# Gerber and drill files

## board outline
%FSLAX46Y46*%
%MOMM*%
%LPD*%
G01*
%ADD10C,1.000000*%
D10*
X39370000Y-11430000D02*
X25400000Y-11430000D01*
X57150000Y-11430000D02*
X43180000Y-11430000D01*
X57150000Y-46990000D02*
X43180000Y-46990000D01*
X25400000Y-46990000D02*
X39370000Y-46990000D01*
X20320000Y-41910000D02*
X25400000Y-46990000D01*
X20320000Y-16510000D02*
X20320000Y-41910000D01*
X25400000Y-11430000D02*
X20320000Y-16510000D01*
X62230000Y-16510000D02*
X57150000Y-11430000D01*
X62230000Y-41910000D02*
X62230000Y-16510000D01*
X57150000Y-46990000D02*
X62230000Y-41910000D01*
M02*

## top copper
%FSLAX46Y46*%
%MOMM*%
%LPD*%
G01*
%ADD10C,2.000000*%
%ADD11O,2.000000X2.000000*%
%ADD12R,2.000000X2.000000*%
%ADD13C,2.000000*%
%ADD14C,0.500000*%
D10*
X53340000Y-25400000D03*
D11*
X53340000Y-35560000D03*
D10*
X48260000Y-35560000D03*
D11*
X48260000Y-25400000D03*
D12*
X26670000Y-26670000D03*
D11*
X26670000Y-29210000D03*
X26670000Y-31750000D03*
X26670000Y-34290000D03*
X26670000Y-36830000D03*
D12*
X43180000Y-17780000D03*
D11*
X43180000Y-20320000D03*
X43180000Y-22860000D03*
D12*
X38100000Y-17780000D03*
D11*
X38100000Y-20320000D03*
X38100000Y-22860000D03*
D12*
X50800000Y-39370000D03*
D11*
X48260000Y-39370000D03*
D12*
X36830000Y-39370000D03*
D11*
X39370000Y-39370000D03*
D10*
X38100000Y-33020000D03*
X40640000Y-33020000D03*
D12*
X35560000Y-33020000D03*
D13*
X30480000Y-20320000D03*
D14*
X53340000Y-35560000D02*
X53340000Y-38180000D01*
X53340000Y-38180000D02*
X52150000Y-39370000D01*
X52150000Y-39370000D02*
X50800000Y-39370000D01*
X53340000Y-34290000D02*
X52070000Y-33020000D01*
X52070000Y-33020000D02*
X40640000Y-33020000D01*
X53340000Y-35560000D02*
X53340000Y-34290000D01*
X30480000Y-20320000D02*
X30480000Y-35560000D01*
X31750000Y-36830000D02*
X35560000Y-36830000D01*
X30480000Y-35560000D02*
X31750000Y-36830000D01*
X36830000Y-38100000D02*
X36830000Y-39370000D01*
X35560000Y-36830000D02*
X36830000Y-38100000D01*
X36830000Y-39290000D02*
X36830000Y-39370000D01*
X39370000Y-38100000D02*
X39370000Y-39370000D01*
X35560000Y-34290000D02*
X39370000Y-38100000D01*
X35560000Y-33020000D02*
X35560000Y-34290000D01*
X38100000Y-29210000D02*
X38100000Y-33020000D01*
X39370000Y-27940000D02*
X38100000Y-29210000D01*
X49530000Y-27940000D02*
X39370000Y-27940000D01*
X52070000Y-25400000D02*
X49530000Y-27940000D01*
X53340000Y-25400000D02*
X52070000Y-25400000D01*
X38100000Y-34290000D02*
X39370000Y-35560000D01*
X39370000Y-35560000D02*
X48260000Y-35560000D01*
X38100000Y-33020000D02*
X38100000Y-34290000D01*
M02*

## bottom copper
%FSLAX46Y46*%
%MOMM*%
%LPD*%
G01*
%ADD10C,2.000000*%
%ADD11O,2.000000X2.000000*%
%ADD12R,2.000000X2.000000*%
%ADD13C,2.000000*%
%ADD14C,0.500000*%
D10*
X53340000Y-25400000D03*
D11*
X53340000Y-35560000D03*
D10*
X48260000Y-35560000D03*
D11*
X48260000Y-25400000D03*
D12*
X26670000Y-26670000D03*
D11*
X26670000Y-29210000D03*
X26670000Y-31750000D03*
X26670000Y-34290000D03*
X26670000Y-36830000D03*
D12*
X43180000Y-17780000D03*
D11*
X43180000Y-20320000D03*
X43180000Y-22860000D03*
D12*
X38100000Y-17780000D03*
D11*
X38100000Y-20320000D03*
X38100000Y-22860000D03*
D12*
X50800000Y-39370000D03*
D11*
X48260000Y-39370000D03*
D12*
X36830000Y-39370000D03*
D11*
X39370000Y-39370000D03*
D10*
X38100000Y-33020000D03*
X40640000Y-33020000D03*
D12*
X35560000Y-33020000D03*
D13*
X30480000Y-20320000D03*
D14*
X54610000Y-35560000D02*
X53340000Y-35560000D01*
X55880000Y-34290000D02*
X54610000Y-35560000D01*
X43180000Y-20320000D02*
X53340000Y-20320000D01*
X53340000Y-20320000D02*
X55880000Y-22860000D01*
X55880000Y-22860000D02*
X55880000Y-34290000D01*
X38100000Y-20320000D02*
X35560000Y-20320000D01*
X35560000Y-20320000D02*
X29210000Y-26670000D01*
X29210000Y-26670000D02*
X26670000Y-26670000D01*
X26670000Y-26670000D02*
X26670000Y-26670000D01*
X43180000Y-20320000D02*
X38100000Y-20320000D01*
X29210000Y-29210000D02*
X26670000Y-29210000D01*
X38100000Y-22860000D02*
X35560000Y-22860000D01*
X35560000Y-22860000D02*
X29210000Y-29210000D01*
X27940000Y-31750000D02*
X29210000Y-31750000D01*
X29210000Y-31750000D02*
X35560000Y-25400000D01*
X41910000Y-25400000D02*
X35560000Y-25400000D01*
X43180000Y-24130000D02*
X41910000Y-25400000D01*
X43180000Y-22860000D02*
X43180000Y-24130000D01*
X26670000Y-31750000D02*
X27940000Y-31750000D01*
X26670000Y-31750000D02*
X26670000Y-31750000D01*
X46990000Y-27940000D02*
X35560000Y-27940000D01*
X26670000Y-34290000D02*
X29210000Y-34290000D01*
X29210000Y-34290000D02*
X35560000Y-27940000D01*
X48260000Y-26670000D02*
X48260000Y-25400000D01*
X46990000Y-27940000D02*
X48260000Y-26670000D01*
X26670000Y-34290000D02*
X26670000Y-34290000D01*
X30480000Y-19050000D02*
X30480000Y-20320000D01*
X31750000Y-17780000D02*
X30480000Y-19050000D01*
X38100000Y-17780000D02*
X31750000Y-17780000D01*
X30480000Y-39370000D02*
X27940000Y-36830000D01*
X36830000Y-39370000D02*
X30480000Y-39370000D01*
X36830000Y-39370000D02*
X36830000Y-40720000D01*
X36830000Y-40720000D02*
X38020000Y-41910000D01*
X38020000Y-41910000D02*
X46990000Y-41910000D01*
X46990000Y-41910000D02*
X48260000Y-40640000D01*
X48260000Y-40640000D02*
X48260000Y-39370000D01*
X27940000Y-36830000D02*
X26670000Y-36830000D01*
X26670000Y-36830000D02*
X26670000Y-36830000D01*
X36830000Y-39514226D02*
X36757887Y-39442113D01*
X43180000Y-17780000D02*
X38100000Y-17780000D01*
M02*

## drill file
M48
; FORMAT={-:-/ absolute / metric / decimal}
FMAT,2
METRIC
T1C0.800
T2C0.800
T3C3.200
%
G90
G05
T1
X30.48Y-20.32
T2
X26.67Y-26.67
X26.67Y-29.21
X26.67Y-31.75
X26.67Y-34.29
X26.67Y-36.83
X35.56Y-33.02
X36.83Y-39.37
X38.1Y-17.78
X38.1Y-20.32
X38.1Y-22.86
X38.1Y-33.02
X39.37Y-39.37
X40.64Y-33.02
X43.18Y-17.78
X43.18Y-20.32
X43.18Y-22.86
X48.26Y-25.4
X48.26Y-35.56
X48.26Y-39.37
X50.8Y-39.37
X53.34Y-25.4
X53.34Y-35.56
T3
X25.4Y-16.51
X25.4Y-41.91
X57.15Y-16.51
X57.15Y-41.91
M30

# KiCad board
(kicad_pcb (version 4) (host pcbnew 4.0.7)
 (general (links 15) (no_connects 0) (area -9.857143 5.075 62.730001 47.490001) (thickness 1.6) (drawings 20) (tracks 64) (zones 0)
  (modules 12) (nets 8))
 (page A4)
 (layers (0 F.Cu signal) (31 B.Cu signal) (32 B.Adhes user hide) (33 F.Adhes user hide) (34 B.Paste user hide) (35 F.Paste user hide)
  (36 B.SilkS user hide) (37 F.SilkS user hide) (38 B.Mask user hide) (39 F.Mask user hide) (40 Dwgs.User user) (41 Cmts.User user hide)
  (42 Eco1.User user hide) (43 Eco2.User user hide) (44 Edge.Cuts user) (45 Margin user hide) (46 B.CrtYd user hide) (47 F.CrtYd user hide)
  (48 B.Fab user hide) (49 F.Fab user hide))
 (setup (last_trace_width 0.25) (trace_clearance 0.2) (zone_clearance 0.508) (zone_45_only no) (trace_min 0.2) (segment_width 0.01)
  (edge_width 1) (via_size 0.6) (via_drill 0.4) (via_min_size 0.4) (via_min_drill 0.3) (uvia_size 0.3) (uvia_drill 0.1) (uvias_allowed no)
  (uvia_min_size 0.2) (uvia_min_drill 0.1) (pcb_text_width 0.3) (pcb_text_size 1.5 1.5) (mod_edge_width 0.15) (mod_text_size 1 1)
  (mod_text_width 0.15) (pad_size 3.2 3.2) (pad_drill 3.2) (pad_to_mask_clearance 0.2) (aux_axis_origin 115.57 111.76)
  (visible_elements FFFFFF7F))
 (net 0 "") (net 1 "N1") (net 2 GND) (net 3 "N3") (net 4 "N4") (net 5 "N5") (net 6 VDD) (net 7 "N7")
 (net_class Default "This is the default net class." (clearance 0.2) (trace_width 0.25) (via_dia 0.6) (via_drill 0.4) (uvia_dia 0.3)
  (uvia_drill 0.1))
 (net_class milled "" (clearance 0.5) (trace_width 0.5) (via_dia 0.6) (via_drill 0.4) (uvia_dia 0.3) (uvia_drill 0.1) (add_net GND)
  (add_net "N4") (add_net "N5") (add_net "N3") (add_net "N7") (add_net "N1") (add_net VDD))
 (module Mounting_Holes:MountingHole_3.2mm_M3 (layer F.Cu) (at 57.15 16.51)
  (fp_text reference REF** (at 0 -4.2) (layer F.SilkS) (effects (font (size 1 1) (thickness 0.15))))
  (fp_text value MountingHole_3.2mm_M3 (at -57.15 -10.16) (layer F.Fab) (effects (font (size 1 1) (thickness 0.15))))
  (pad "" np_thru_hole circle (at 0 0) (size 3.2 3.2) (drill 3.2) (layers *.Cu *.Mask)))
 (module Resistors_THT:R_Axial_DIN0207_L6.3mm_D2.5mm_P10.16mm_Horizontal (layer F.Cu) (at 53.34 25.4 270)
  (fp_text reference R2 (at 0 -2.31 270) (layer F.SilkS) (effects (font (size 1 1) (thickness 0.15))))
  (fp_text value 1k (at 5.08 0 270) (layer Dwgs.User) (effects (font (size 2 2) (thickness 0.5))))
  (pad 1 thru_hole circle (at 0 0 270) (size 2 2) (drill 0.8) (layers *.Cu *.Mask) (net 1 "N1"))
  (pad 2 thru_hole oval (at 10.16 0 270) (size 2 2) (drill 0.8) (layers *.Cu *.Mask) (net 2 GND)))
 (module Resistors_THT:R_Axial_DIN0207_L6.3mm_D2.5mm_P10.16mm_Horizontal (layer F.Cu) (at 48.26 35.56 90)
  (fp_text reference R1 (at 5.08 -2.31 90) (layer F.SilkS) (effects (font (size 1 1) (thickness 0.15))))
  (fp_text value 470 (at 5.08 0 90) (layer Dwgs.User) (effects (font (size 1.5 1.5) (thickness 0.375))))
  (pad 1 thru_hole circle (at 0 0 90) (size 2 2) (drill 0.8) (layers *.Cu *.Mask) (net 1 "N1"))
  (pad 2 thru_hole oval (at 10.16 0 90) (size 2 2) (drill 0.8) (layers *.Cu *.Mask) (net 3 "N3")))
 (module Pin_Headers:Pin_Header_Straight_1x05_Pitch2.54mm (layer F.Cu) (at 26.67 26.67)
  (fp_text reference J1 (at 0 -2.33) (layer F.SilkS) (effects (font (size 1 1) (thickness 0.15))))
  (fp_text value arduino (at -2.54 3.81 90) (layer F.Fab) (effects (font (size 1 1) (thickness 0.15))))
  (pad 1 thru_hole rect (at 0 0) (size 2 2) (drill 0.8) (layers *.Cu *.Mask) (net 2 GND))
  (pad 2 thru_hole oval (at 0 2.54) (size 2 2) (drill 0.8) (layers *.Cu *.Mask) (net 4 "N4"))
  (pad 3 thru_hole oval (at 0 5.08) (size 2 2) (drill 0.8) (layers *.Cu *.Mask) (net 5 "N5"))
  (pad 4 thru_hole oval (at 0 7.62) (size 2 2) (drill 0.8) (layers *.Cu *.Mask) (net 3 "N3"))
  (pad 5 thru_hole oval (at 0 10.16) (size 2 2) (drill 0.8) (layers *.Cu *.Mask) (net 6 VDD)))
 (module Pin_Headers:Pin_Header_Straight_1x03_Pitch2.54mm (layer F.Cu) (at 43.18 17.78)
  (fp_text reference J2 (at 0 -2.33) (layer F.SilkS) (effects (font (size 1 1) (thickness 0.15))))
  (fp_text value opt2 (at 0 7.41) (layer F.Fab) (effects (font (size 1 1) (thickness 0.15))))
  (pad 1 thru_hole rect (at 0 0) (size 2 2) (drill 0.8) (layers *.Cu *.Mask) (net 6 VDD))
  (pad 2 thru_hole oval (at 0 2.54) (size 2 2) (drill 0.8) (layers *.Cu *.Mask) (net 2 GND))
  (pad 3 thru_hole oval (at 0 5.08) (size 2 2) (drill 0.8) (layers *.Cu *.Mask) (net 5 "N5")))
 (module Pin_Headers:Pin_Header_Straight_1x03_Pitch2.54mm (layer F.Cu) (at 38.1 17.78)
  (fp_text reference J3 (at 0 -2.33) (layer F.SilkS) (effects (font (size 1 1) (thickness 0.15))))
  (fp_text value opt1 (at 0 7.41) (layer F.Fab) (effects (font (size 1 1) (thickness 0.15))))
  (pad 1 thru_hole rect (at 0 0) (size 2 2) (drill 0.8) (layers *.Cu *.Mask) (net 6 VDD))
  (pad 2 thru_hole oval (at 0 2.54) (size 2 2) (drill 0.8) (layers *.Cu *.Mask) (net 2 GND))
  (pad 3 thru_hole oval (at 0 5.08) (size 2 2) (drill 0.8) (layers *.Cu *.Mask) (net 4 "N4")))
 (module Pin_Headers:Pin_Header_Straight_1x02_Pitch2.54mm (layer F.Cu) (at 50.8 39.37 270)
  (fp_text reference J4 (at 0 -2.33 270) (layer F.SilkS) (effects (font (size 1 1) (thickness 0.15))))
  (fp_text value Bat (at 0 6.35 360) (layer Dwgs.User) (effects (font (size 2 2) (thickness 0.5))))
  (pad 1 thru_hole rect (at 0 0 270) (size 2 2) (drill 0.8) (layers *.Cu *.Mask) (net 2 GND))
  (pad 2 thru_hole oval (at 0 2.54 270) (size 2 2) (drill 0.8) (layers *.Cu *.Mask) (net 6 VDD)))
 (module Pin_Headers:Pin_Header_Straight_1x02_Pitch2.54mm (layer F.Cu) (at 36.83 39.37 90)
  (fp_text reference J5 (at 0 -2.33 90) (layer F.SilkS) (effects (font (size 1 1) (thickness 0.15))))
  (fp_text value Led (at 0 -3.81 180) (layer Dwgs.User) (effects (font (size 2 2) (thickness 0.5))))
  (pad 1 thru_hole rect (at 0 0 90) (size 2 2) (drill 0.8) (layers *.Cu *.Mask) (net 6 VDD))
  (pad 2 thru_hole oval (at 0 2.54 90) (size 2 2) (drill 0.8) (layers *.Cu *.Mask) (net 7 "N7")))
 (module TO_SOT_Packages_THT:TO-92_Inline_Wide (layer F.Cu) (at 35.56 33.02)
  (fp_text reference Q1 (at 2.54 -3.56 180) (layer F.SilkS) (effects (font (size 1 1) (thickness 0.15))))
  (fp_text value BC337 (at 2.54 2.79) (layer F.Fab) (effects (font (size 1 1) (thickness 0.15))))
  (pad 2 thru_hole circle (at 2.54 0 90) (size 2 2) (drill 0.8) (layers *.Cu *.Mask) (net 1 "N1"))
  (pad 3 thru_hole circle (at 5.08 0 90) (size 2 2) (drill 0.8) (layers *.Cu *.Mask) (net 2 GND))
  (pad 1 thru_hole rect (at 0 0 90) (size 2 2) (drill 0.8) (layers *.Cu *.Mask) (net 7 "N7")))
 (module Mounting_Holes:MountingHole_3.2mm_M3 (layer F.Cu) (at 57.15 41.91)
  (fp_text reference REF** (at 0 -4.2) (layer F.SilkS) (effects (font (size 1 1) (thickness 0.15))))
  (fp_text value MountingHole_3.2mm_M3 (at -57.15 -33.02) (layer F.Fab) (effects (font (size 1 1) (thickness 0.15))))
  (pad "" np_thru_hole circle (at 0 0) (size 3.2 3.2) (drill 3.2) (layers *.Cu *.Mask)))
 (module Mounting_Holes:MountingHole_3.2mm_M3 (layer F.Cu) (at 25.4 41.91)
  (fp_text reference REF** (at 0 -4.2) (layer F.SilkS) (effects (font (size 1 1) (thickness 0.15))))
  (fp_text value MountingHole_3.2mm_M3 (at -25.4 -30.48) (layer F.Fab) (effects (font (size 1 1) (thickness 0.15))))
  (pad "" np_thru_hole circle (at 0 0) (size 3.2 3.2) (drill 3.2) (layers *.Cu *.Mask)))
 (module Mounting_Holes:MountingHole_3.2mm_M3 (layer F.Cu) (at 25.4 16.51)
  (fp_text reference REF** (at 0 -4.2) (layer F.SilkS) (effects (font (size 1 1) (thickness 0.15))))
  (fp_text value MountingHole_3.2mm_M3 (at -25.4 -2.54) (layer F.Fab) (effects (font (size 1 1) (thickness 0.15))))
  (pad "" np_thru_hole circle (at 0 0) (size 3.2 3.2) (drill 3.2) (layers *.Cu *.Mask)))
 (gr_line (start 39.37 11.43) (end 25.4 11.43) (layer Edge.Cuts) (width 1))
 (gr_line (start 57.15 11.43) (end 43.18 11.43) (layer Edge.Cuts) (width 1))
 (gr_line (start 57.15 46.99) (end 43.18 46.99) (layer Edge.Cuts) (width 1))
 (gr_line (start 25.4 46.99) (end 39.37 46.99) (layer Edge.Cuts) (width 1))
 (gr_line (start 20.32 41.91) (end 25.4 46.99) (layer Edge.Cuts) (width 1))
 (gr_line (start 20.32 16.51) (end 20.32 41.91) (layer Edge.Cuts) (width 1))
 (gr_line (start 25.4 11.43) (end 20.32 16.51) (layer Edge.Cuts) (width 1))
 (gr_line (start 62.23 16.51) (end 57.15 11.43) (layer Edge.Cuts) (width 1))
 (gr_line (start 62.23 41.91) (end 62.23 16.51) (layer Edge.Cuts) (width 1))
 (gr_line (start 57.15 46.99) (end 62.23 41.91) (layer Edge.Cuts) (width 1))
 (segment (start 54.61 35.56) (end 53.34 35.56) (width 0.5) (layer B.Cu) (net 2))
 (segment (start 55.88 34.29) (end 54.61 35.56) (width 0.5) (layer B.Cu) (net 2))
 (segment (start 43.18 20.32) (end 53.34 20.32) (width 0.5) (layer B.Cu) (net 2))
 (segment (start 53.34 20.32) (end 55.88 22.86) (width 0.5) (layer B.Cu) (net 2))
 (segment (start 55.88 22.86) (end 55.88 34.29) (width 0.5) (layer B.Cu) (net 2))
 (segment (start 53.34 35.56) (end 53.34 38.18) (width 0.5) (layer F.Cu) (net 2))
 (segment (start 53.34 38.18) (end 52.15 39.37) (width 0.5) (layer F.Cu) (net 2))
 (segment (start 52.15 39.37) (end 50.8 39.37) (width 0.5) (layer F.Cu) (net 2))
 (segment (start 53.34 34.29) (end 52.07 33.02) (width 0.5) (layer F.Cu) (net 2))
 (segment (start 52.07 33.02) (end 40.64 33.02) (width 0.5) (layer F.Cu) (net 2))
 (segment (start 53.34 35.56) (end 53.34 34.29) (width 0.5) (layer F.Cu) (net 2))
 (segment (start 38.1 20.32) (end 35.56 20.32) (width 0.5) (layer B.Cu) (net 2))
 (segment (start 35.56 20.32) (end 29.21 26.67) (width 0.5) (layer B.Cu) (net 2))
 (segment (start 29.21 26.67) (end 26.67 26.67) (width 0.5) (layer B.Cu) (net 2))
 (segment (start 26.67 26.67) (end 26.67 26.67) (width 0.5) (layer B.Cu) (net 2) (status 30))
 (segment (start 43.18 20.32) (end 38.1 20.32) (width 0.5) (layer B.Cu) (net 2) (status 20))
 (segment (start 29.21 29.21) (end 26.67 29.21) (width 0.5) (layer B.Cu) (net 4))
 (segment (start 38.1 22.86) (end 35.56 22.86) (width 0.5) (layer B.Cu) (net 4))
 (segment (start 35.56 22.86) (end 29.21 29.21) (width 0.5) (layer B.Cu) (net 4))
 (segment (start 27.94 31.75) (end 29.21 31.75) (width 0.5) (layer B.Cu) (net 5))
 (segment (start 29.21 31.75) (end 35.56 25.4) (width 0.5) (layer B.Cu) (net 5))
 (segment (start 41.91 25.4) (end 35.56 25.4) (width 0.5) (layer B.Cu) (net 5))
 (segment (start 43.18 24.13) (end 41.91 25.4) (width 0.5) (layer B.Cu) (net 5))
 (segment (start 43.18 22.86) (end 43.18 24.13) (width 0.5) (layer B.Cu) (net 5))
 (segment (start 26.67 31.75) (end 27.94 31.75) (width 0.5) (layer B.Cu) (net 5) (status 10))
 (segment (start 26.67 31.75) (end 26.67 31.75) (width 0.5) (layer B.Cu) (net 5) (status 30))
 (segment (start 46.99 27.94) (end 35.56 27.94) (width 0.5) (layer B.Cu) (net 3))
 (segment (start 26.67 34.29) (end 29.21 34.29) (width 0.5) (layer B.Cu) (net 3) (status 10))
 (segment (start 29.21 34.29) (end 35.56 27.94) (width 0.5) (layer B.Cu) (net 3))
 (segment (start 48.26 26.67) (end 48.26 25.4) (width 0.5) (layer B.Cu) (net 3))
 (segment (start 46.99 27.94) (end 48.26 26.67) (width 0.5) (layer B.Cu) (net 3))
 (segment (start 26.67 34.29) (end 26.67 34.29) (width 0.5) (layer B.Cu) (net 3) (status 30))
 (segment (start 30.48 20.32) (end 30.48 35.56) (width 0.5) (layer F.Cu) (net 6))
 (segment (start 30.48 19.05) (end 30.48 20.32) (width 0.5) (layer B.Cu) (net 6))
 (via (at 30.48 20.32) (size 2) (drill 0.8) (layers F.Cu B.Cu) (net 6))
 (segment (start 31.75 17.78) (end 30.48 19.05) (width 0.5) (layer B.Cu) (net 6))
 (segment (start 38.1 17.78) (end 31.75 17.78) (width 0.5) (layer B.Cu) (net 6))
 (segment (start 31.75 36.83) (end 35.56 36.83) (width 0.5) (layer F.Cu) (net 6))
 (segment (start 30.48 35.56) (end 31.75 36.83) (width 0.5) (layer F.Cu) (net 6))
 (segment (start 36.83 38.1) (end 36.83 39.37) (width 0.5) (layer F.Cu) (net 6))
 (segment (start 35.56 36.83) (end 36.83 38.1) (width 0.5) (layer F.Cu) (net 6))
 (segment (start 30.48 39.37) (end 27.94 36.83) (width 0.5) (layer B.Cu) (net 6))
 (segment (start 36.83 39.37) (end 30.48 39.37) (width 0.5) (layer B.Cu) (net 6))
 (segment (start 36.83 39.37) (end 36.83 40.72) (width 0.5) (layer B.Cu) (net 6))
 (segment (start 36.83 40.72) (end 38.02 41.91) (width 0.5) (layer B.Cu) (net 6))
 (segment (start 38.02 41.91) (end 46.99 41.91) (width 0.5) (layer B.Cu) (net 6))
 (segment (start 46.99 41.91) (end 48.26 40.64) (width 0.5) (layer B.Cu) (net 6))
 (segment (start 48.26 40.64) (end 48.26 39.37) (width 0.5) (layer B.Cu) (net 6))
 (segment (start 27.94 36.83) (end 26.67 36.83) (width 0.5) (layer B.Cu) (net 6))
 (segment (start 26.67 36.83) (end 26.67 36.83) (width 0.5) (layer B.Cu) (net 6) (status 20))
 (segment (start 36.83 39.514226) (end 36.757887 39.442113) (width 0.5) (layer B.Cu) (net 6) (status 30))
 (segment (start 36.83 39.29) (end 36.83 39.37) (width 0.5) (layer F.Cu) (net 6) (status 30))
 (segment (start 43.18 17.78) (end 38.1 17.78) (width 0.5) (layer B.Cu) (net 6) (status 20))
 (segment (start 39.37 38.1) (end 39.37 39.37) (width 0.5) (layer F.Cu) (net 7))
 (segment (start 35.56 34.29) (end 39.37 38.1) (width 0.5) (layer F.Cu) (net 7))
 (segment (start 35.56 33.02) (end 35.56 34.29) (width 0.5) (layer F.Cu) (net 7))
 (segment (start 38.1 29.21) (end 38.1 33.02) (width 0.5) (layer F.Cu) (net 1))
 (segment (start 39.37 27.94) (end 38.1 29.21) (width 0.5) (layer F.Cu) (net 1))
 (segment (start 49.53 27.94) (end 39.37 27.94) (width 0.5) (layer F.Cu) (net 1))
 (segment (start 52.07 25.4) (end 49.53 27.94) (width 0.5) (layer F.Cu) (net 1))
 (segment (start 53.34 25.4) (end 52.07 25.4) (width 0.5) (layer F.Cu) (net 1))
 (segment (start 38.1 34.29) (end 39.37 35.56) (width 0.5) (layer F.Cu) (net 1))
 (segment (start 39.37 35.56) (end 48.26 35.56) (width 0.5) (layer F.Cu) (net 1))
 (segment (start 38.1 33.02) (end 38.1 34.29) (width 0.5) (layer F.Cu) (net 1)))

